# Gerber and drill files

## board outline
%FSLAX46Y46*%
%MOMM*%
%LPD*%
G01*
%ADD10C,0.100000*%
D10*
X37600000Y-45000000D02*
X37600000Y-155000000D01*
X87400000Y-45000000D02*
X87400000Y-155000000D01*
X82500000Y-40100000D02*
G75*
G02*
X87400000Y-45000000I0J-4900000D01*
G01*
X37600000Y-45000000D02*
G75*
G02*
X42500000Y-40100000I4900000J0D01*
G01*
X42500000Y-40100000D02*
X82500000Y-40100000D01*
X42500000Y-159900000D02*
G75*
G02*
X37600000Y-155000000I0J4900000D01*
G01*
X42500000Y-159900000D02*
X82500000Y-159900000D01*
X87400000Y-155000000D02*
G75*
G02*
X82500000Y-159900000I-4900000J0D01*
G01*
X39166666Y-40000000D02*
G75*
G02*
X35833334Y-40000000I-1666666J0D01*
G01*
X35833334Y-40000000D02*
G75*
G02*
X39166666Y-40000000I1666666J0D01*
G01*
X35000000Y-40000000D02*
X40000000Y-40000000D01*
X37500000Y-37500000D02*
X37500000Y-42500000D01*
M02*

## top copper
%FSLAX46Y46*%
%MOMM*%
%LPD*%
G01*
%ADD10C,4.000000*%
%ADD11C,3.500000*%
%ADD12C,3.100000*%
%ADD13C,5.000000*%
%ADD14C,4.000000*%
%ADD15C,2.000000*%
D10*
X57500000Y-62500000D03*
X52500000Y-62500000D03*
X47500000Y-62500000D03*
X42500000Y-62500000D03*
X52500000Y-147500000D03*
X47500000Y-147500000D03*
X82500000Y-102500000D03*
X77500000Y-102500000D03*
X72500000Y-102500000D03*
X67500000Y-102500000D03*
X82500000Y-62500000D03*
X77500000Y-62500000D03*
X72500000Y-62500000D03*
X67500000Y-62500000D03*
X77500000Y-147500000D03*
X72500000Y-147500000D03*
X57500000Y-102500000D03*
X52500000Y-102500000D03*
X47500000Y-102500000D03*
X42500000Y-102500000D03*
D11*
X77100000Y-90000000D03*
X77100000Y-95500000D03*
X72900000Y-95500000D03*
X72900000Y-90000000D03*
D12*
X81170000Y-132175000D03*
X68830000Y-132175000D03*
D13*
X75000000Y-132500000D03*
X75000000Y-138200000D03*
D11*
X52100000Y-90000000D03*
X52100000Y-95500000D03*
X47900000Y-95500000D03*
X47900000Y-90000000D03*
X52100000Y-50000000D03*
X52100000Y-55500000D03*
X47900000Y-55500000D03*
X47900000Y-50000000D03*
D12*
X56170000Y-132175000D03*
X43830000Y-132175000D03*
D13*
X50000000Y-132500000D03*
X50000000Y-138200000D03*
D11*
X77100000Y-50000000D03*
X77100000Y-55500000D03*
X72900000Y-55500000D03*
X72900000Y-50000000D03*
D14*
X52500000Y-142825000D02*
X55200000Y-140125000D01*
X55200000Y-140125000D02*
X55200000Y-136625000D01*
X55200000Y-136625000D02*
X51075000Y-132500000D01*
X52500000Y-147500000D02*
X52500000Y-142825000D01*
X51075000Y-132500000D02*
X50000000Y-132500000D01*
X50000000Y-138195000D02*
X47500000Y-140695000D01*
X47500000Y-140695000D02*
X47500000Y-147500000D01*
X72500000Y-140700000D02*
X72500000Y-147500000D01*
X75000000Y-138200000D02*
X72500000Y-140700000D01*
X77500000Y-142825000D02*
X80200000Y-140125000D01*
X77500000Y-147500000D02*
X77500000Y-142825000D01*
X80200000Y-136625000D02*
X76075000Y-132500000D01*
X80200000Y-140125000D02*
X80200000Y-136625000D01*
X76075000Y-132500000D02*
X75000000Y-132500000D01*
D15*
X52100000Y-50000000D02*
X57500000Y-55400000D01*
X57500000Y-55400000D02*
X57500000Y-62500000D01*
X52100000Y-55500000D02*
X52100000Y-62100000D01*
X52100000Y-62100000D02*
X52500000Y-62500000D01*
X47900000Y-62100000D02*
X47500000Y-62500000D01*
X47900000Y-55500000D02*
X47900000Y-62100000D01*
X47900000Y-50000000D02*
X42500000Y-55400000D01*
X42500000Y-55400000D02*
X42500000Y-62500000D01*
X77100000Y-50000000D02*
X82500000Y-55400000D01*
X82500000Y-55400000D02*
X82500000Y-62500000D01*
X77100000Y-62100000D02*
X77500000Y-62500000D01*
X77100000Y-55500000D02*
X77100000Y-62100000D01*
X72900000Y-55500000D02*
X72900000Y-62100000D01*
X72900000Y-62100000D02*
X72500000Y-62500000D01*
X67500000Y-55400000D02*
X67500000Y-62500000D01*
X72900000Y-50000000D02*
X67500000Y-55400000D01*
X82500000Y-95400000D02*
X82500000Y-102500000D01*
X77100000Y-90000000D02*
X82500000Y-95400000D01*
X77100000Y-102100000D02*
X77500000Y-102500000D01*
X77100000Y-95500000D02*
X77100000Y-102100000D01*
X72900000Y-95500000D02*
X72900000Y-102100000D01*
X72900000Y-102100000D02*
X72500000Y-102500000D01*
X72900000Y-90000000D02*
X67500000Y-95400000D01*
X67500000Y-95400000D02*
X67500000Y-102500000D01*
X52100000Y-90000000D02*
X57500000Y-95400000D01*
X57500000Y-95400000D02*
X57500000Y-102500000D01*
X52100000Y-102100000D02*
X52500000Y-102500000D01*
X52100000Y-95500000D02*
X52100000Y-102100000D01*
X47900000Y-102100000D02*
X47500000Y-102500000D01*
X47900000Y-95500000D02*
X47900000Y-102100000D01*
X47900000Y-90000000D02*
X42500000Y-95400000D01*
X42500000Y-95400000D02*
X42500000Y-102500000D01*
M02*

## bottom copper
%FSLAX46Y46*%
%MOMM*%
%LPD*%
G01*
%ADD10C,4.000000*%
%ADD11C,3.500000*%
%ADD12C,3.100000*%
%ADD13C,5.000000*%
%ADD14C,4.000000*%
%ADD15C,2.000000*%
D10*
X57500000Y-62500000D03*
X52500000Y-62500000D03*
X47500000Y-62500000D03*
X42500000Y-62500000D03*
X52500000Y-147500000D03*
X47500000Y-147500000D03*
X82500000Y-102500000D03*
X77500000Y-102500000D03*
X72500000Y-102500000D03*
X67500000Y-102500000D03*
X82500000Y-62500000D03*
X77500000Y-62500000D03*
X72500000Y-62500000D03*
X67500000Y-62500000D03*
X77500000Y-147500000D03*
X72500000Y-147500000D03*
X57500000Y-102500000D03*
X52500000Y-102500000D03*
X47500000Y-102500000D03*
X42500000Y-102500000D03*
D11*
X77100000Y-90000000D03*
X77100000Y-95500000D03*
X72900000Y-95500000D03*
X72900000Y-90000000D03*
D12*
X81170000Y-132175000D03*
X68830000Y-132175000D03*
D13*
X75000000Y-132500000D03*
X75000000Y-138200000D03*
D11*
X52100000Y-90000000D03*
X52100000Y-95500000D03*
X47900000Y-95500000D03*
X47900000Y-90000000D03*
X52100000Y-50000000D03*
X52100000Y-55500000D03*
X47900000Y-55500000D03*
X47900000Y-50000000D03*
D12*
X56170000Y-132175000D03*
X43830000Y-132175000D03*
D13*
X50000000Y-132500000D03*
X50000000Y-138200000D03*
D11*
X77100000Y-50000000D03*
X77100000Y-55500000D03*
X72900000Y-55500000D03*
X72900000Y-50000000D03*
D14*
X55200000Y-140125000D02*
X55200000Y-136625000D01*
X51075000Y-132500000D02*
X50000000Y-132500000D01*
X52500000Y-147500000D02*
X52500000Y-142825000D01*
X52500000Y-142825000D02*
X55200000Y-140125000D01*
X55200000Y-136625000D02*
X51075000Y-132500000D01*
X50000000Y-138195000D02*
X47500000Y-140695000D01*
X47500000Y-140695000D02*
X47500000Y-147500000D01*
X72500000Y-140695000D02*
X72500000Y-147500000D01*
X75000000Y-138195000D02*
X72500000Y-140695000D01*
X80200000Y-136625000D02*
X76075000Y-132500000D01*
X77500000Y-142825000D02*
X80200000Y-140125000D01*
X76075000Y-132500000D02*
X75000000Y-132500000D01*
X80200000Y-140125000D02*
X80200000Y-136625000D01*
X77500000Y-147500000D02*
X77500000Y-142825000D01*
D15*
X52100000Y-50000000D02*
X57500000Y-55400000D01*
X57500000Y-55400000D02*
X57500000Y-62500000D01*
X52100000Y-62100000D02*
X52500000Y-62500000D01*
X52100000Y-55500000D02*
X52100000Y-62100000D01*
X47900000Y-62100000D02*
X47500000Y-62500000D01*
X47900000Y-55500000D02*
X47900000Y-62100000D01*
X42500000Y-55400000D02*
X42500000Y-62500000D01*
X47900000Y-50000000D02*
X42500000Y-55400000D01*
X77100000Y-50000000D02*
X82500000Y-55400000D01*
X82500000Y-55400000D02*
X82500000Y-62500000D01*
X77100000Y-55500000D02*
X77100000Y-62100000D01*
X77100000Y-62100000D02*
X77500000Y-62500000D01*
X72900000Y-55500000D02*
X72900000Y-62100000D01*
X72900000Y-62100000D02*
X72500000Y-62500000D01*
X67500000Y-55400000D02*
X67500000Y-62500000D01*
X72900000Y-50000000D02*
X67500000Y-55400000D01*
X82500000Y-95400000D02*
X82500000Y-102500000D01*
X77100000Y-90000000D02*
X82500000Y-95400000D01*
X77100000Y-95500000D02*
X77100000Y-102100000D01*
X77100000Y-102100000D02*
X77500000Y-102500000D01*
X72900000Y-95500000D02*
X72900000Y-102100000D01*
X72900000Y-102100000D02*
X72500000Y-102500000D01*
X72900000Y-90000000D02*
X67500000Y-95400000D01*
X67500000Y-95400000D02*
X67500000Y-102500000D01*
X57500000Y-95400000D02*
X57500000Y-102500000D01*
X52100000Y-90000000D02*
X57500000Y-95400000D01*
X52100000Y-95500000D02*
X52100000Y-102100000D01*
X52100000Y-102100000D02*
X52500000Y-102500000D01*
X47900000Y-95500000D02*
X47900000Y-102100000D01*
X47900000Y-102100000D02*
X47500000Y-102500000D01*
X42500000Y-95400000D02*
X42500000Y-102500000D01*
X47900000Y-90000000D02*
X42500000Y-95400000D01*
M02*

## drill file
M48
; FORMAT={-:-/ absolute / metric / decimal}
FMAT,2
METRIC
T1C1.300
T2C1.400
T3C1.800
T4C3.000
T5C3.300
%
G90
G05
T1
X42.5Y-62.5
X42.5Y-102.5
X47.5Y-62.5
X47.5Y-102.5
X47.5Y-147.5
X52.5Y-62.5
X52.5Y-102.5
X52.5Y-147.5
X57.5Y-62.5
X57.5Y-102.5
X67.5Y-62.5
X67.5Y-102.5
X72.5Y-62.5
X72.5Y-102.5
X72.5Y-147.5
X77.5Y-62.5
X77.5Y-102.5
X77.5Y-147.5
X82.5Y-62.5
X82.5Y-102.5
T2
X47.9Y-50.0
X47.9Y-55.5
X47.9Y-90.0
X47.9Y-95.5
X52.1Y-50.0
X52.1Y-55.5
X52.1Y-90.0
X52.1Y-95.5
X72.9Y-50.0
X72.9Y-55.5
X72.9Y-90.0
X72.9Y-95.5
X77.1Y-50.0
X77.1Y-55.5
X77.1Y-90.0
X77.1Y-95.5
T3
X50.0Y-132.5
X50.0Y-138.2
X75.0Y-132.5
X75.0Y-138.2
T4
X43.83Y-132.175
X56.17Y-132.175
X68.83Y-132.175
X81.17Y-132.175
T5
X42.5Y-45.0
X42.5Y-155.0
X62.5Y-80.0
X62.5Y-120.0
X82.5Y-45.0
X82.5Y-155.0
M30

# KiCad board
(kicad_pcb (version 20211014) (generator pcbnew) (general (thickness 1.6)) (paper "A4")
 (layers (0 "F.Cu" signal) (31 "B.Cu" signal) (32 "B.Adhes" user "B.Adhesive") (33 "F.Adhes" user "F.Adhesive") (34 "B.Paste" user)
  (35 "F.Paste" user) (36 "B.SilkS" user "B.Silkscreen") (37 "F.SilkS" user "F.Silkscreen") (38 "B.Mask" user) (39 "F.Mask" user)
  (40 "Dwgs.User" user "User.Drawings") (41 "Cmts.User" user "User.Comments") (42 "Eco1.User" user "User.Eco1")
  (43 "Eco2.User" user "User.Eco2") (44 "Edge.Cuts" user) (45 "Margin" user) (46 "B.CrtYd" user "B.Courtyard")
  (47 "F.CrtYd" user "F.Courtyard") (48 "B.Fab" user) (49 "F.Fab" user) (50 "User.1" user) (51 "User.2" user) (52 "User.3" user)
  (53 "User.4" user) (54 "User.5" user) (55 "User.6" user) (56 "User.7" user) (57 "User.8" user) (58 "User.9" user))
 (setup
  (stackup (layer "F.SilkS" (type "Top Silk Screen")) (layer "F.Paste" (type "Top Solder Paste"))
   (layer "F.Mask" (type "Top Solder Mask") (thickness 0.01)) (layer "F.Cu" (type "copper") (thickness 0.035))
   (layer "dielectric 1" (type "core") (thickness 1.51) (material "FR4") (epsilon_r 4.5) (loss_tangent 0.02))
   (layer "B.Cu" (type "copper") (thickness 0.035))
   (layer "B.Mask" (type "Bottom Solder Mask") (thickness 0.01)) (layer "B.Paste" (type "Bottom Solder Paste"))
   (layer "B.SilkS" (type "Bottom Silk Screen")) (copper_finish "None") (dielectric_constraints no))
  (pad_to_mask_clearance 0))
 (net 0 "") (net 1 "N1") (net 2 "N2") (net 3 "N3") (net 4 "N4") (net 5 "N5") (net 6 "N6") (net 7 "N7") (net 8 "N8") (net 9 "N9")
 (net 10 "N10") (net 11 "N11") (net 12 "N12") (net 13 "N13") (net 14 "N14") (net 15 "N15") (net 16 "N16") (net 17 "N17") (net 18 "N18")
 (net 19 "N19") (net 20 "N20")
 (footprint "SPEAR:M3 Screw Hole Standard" (layer "F.Cu") (at 62.5 120)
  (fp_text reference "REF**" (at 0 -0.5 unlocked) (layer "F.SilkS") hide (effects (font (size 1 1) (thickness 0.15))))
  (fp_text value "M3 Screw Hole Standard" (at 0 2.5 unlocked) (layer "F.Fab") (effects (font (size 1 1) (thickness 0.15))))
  (pad "" np_thru_hole circle (at 0 0) (size 3.3 3.3) (drill 3.3) (layers F&B.Cu *.Mask)))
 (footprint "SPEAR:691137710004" (layer "F.Cu") (at 50 62.5)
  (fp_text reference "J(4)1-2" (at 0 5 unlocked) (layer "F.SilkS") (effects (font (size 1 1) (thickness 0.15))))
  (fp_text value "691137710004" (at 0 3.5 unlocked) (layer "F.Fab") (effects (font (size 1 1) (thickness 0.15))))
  (pad "1" thru_hole circle (at 7.5 0) (size 4 4) (drill 1.3) (layers *.Cu *.Mask) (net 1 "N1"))
  (pad "2" thru_hole circle (at 2.5 0) (size 4 4) (drill 1.3) (layers *.Cu *.Mask) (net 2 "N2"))
  (pad "3" thru_hole circle (at -2.5 0) (size 4 4) (drill 1.3) (layers *.Cu *.Mask) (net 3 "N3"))
  (pad "4" thru_hole circle (at -7.5 0) (size 4 4) (drill 1.3) (layers *.Cu *.Mask) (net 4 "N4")))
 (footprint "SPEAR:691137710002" (layer "F.Cu") (at 50 147.5)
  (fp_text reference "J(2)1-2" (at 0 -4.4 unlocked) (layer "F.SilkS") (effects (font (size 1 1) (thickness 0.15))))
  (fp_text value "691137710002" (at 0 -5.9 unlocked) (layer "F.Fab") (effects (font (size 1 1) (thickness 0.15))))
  (pad "1" thru_hole circle (at 2.5 0) (size 4 4) (drill 1.3) (layers *.Cu *.Mask) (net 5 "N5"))
  (pad "2" thru_hole circle (at -2.5 0) (size 4 4) (drill 1.3) (layers *.Cu *.Mask) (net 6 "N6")))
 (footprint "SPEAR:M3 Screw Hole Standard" (layer "F.Cu") (at 42.5 155)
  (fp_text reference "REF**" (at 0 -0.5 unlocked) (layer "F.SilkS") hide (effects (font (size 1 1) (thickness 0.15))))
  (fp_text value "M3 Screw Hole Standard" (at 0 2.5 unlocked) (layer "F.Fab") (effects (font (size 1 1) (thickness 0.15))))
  (pad "" np_thru_hole circle (at 0 0) (size 3.3 3.3) (drill 3.3) (layers F&B.Cu *.Mask)))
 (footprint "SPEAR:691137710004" (layer "F.Cu") (at 75 102.5)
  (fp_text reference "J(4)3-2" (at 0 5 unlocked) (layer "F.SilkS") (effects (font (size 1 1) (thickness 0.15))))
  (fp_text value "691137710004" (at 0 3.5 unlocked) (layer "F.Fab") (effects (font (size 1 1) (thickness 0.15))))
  (pad "1" thru_hole circle (at 7.5 0) (size 4 4) (drill 1.3) (layers *.Cu *.Mask) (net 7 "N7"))
  (pad "2" thru_hole circle (at 2.5 0) (size 4 4) (drill 1.3) (layers *.Cu *.Mask) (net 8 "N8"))
  (pad "3" thru_hole circle (at -2.5 0) (size 4 4) (drill 1.3) (layers *.Cu *.Mask) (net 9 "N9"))
  (pad "4" thru_hole circle (at -7.5 0) (size 4 4) (drill 1.3) (layers *.Cu *.Mask) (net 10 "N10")))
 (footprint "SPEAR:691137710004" (layer "F.Cu") (at 75 62.5)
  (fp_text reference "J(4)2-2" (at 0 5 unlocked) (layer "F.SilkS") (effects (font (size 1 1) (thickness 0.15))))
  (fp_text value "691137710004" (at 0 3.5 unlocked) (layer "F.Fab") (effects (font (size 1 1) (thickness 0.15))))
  (pad "1" thru_hole circle (at 7.5 0) (size 4 4) (drill 1.3) (layers *.Cu *.Mask) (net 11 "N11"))
  (pad "2" thru_hole circle (at 2.5 0) (size 4 4) (drill 1.3) (layers *.Cu *.Mask) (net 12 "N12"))
  (pad "3" thru_hole circle (at -2.5 0) (size 4 4) (drill 1.3) (layers *.Cu *.Mask) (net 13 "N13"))
  (pad "4" thru_hole circle (at -7.5 0) (size 4 4) (drill 1.3) (layers *.Cu *.Mask) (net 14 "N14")))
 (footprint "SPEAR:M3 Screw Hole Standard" (layer "F.Cu") (at 62.5 80)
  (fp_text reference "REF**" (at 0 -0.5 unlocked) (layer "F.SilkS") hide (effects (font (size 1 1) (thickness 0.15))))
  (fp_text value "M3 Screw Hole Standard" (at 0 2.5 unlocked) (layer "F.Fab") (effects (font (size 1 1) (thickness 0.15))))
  (pad "" np_thru_hole circle (at 0 0) (size 3.3 3.3) (drill 3.3) (layers F&B.Cu *.Mask)))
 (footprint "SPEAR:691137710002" (layer "F.Cu") (at 75 147.5)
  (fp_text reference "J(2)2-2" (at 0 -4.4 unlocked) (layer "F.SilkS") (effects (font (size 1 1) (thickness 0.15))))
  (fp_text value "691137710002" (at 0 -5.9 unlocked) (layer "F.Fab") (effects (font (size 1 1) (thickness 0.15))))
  (pad "1" thru_hole circle (at 2.5 0) (size 4 4) (drill 1.3) (layers *.Cu *.Mask) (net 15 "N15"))
  (pad "2" thru_hole circle (at -2.5 0) (size 4 4) (drill 1.3) (layers *.Cu *.Mask) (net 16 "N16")))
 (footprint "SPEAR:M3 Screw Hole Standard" (layer "F.Cu") (at 82.5 45)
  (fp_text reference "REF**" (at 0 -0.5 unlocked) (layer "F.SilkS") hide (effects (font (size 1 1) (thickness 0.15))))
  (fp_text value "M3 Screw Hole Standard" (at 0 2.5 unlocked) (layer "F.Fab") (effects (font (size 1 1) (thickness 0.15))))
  (pad "" np_thru_hole circle (at 0 0) (size 3.3 3.3) (drill 3.3) (layers F&B.Cu *.Mask)))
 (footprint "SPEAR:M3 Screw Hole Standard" (layer "F.Cu") (at 42.5 45)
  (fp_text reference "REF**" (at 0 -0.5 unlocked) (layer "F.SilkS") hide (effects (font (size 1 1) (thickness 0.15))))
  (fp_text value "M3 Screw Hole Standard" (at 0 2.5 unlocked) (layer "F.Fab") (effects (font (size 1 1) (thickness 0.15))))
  (pad "" np_thru_hole circle (at 0 0) (size 3.3 3.3) (drill 3.3) (layers F&B.Cu *.Mask)))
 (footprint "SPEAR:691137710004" (layer "F.Cu") (at 50 102.5)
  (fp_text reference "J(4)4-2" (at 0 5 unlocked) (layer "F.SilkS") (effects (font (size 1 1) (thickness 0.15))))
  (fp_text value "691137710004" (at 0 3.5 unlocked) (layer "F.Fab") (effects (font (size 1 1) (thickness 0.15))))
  (pad "1" thru_hole circle (at 7.5 0) (size 4 4) (drill 1.3) (layers *.Cu *.Mask) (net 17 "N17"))
  (pad "2" thru_hole circle (at 2.5 0) (size 4 4) (drill 1.3) (layers *.Cu *.Mask) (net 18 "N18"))
  (pad "3" thru_hole circle (at -2.5 0) (size 4 4) (drill 1.3) (layers *.Cu *.Mask) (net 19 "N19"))
  (pad "4" thru_hole circle (at -7.5 0) (size 4 4) (drill 1.3) (layers *.Cu *.Mask) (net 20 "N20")))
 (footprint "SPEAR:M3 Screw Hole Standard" (layer "F.Cu") (at 82.5 155)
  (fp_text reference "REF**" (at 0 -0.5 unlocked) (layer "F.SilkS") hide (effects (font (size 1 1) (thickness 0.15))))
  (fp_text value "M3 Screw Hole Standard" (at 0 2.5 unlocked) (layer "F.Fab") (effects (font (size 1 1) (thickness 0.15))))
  (pad "" np_thru_hole circle (at 0 0) (size 3.3 3.3) (drill 3.3) (layers F&B.Cu *.Mask)))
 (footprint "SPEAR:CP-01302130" (layer "B.Cu") (at 75 90 180)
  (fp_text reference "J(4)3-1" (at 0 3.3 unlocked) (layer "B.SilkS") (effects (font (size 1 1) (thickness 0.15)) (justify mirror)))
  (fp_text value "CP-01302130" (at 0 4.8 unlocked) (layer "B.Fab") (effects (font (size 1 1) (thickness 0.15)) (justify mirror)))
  (pad "1" thru_hole circle (at -2.1 0 180) (size 3.5 3.5) (drill 1.4) (layers *.Cu *.Mask) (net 7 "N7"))
  (pad "2" thru_hole circle (at -2.1 -5.5 180) (size 3.5 3.5) (drill 1.4) (layers *.Cu *.Mask) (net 8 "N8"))
  (pad "3" thru_hole circle (at 2.1 -5.5 180) (size 3.5 3.5) (drill 1.4) (layers *.Cu *.Mask) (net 9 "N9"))
  (pad "4" thru_hole circle (at 2.1 0 180) (size 3.5 3.5) (drill 1.4) (layers *.Cu *.Mask) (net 10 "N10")))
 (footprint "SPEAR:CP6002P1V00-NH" (layer "B.Cu") (at 75 132.5 180)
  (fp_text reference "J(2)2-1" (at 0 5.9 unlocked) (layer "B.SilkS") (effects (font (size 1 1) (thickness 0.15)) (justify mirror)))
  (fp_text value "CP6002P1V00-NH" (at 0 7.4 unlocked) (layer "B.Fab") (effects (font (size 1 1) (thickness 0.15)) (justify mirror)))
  (pad "" np_thru_hole circle (at -6.17 0.325 180) (size 3.1 3.1) (drill 3) (layers F&B.Cu *.Mask))
  (pad "" np_thru_hole circle (at 6.17 0.325 180) (size 3.1 3.1) (drill 3) (layers F&B.Cu *.Mask))
  (pad "1" thru_hole circle (at 0 0 180) (size 5 5) (drill 1.8) (layers *.Cu *.Mask) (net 15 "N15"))
  (pad "2" thru_hole circle (at 0 -5.7 180) (size 5 5) (drill 1.8) (layers *.Cu *.Mask) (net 16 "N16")))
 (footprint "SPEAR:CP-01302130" (layer "B.Cu") (at 50 90 180)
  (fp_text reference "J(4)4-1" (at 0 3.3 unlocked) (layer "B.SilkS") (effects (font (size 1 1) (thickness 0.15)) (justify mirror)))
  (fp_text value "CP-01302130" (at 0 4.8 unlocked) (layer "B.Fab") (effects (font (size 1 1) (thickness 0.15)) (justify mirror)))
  (pad "1" thru_hole circle (at -2.1 0 180) (size 3.5 3.5) (drill 1.4) (layers *.Cu *.Mask) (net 17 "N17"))
  (pad "2" thru_hole circle (at -2.1 -5.5 180) (size 3.5 3.5) (drill 1.4) (layers *.Cu *.Mask) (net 18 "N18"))
  (pad "3" thru_hole circle (at 2.1 -5.5 180) (size 3.5 3.5) (drill 1.4) (layers *.Cu *.Mask) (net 19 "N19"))
  (pad "4" thru_hole circle (at 2.1 0 180) (size 3.5 3.5) (drill 1.4) (layers *.Cu *.Mask) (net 20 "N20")))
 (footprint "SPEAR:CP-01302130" (layer "B.Cu") (at 50 50 180)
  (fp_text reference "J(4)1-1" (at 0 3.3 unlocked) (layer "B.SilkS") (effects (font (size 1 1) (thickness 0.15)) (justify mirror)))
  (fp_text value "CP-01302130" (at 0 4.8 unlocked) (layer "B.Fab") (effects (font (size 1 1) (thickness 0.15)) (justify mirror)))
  (pad "1" thru_hole circle (at -2.1 0 180) (size 3.5 3.5) (drill 1.4) (layers *.Cu *.Mask) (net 1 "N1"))
  (pad "2" thru_hole circle (at -2.1 -5.5 180) (size 3.5 3.5) (drill 1.4) (layers *.Cu *.Mask) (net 2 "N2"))
  (pad "3" thru_hole circle (at 2.1 -5.5 180) (size 3.5 3.5) (drill 1.4) (layers *.Cu *.Mask) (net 3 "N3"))
  (pad "4" thru_hole circle (at 2.1 0 180) (size 3.5 3.5) (drill 1.4) (layers *.Cu *.Mask) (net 4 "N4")))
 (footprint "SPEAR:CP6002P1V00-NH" (layer "B.Cu") (at 50 132.5 180)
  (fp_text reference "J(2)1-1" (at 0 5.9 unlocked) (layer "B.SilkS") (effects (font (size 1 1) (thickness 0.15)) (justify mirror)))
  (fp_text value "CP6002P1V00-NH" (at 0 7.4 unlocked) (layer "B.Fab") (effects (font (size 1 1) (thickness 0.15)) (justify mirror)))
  (pad "" np_thru_hole circle (at -6.17 0.325 180) (size 3.1 3.1) (drill 3) (layers F&B.Cu *.Mask))
  (pad "" np_thru_hole circle (at 6.17 0.325 180) (size 3.1 3.1) (drill 3) (layers F&B.Cu *.Mask))
  (pad "1" thru_hole circle (at 0 0 180) (size 5 5) (drill 1.8) (layers *.Cu *.Mask) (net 5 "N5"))
  (pad "2" thru_hole circle (at 0 -5.7 180) (size 5 5) (drill 1.8) (layers *.Cu *.Mask) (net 6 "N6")))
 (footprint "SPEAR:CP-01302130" (layer "B.Cu") (at 75 50 180)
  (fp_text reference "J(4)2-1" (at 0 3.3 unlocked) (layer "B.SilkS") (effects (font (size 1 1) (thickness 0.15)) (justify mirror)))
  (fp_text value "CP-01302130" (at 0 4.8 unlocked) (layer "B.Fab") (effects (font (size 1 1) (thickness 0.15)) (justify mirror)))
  (pad "1" thru_hole circle (at -2.1 0 180) (size 3.5 3.5) (drill 1.4) (layers *.Cu *.Mask) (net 11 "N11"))
  (pad "2" thru_hole circle (at -2.1 -5.5 180) (size 3.5 3.5) (drill 1.4) (layers *.Cu *.Mask) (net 12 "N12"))
  (pad "3" thru_hole circle (at 2.1 -5.5 180) (size 3.5 3.5) (drill 1.4) (layers *.Cu *.Mask) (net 13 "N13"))
  (pad "4" thru_hole circle (at 2.1 0 180) (size 3.5 3.5) (drill 1.4) (layers *.Cu *.Mask) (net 14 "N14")))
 (gr_line (start 37.6 45) (end 37.6 155) (layer "Edge.Cuts") (width 0.1))
 (gr_line (start 87.4 45) (end 87.4 155) (layer "Edge.Cuts") (width 0.1))
 (gr_arc (start 82.5 40.1) (mid 85.964823 41.535177) (end 87.4 45) (layer "Edge.Cuts") (width 0.1))
 (gr_arc (start 37.6 45) (mid 39.035177 41.535177) (end 42.5 40.1) (layer "Edge.Cuts") (width 0.1))
 (gr_line (start 42.5 40.1) (end 82.5 40.1) (layer "Edge.Cuts") (width 0.1))
 (gr_arc (start 42.5 159.9) (mid 39.035177 158.464823) (end 37.6 155) (layer "Edge.Cuts") (width 0.1))
 (gr_line (start 42.5 159.9) (end 82.5 159.9) (layer "Edge.Cuts") (width 0.1))
 (gr_arc (start 87.4 155) (mid 85.964823 158.464823) (end 82.5 159.9) (layer "Edge.Cuts") (width 0.1))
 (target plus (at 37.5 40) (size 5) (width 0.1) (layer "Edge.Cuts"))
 (segment (start 52.5 142.825) (end 55.2 140.125) (width 4) (layer "F.Cu") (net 5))
 (segment (start 55.2 140.125) (end 55.2 136.625) (width 4) (layer "F.Cu") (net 5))
 (segment (start 55.2 136.625) (end 51.075 132.5) (width 4) (layer "F.Cu") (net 5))
 (segment (start 52.5 147.5) (end 52.5 142.825) (width 4) (layer "F.Cu") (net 5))
 (segment (start 51.075 132.5) (end 50 132.5) (width 4) (layer "F.Cu") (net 5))
 (segment (start 55.2 140.125) (end 55.2 136.625) (width 4) (layer "B.Cu") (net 5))
 (segment (start 51.075 132.5) (end 50 132.5) (width 4) (layer "B.Cu") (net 5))
 (segment (start 52.5 147.5) (end 52.5 142.825) (width 4) (layer "B.Cu") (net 5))
 (segment (start 52.5 142.825) (end 55.2 140.125) (width 4) (layer "B.Cu") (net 5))
 (segment (start 55.2 136.625) (end 51.075 132.5) (width 4) (layer "B.Cu") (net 5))
 (segment (start 50 138.195) (end 47.5 140.695) (width 4) (layer "F.Cu") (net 6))
 (segment (start 47.5 140.695) (end 47.5 147.5) (width 4) (layer "F.Cu") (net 6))
 (segment (start 50 138.195) (end 47.5 140.695) (width 4) (layer "B.Cu") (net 6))
 (segment (start 47.5 140.695) (end 47.5 147.5) (width 4) (layer "B.Cu") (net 6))
 (segment (start 72.5 140.7) (end 72.5 147.5) (width 4) (layer "F.Cu") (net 16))
 (segment (start 75 138.2) (end 72.5 140.7) (width 4) (layer "F.Cu") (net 16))
 (segment (start 72.5 140.695) (end 72.5 147.5) (width 4) (layer "B.Cu") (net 16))
 (segment (start 75 138.195) (end 72.5 140.695) (width 4) (layer "B.Cu") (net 16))
 (segment (start 77.5 142.825) (end 80.2 140.125) (width 4) (layer "F.Cu") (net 15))
 (segment (start 77.5 147.5) (end 77.5 142.825) (width 4) (layer "F.Cu") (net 15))
 (segment (start 80.2 136.625) (end 76.075 132.5) (width 4) (layer "F.Cu") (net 15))
 (segment (start 80.2 140.125) (end 80.2 136.625) (width 4) (layer "F.Cu") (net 15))
 (segment (start 76.075 132.5) (end 75 132.5) (width 4) (layer "F.Cu") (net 15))
 (segment (start 80.2 136.625) (end 76.075 132.5) (width 4) (layer "B.Cu") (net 15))
 (segment (start 77.5 142.825) (end 80.2 140.125) (width 4) (layer "B.Cu") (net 15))
 (segment (start 76.075 132.5) (end 75 132.5) (width 4) (layer "B.Cu") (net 15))
 (segment (start 80.2 140.125) (end 80.2 136.625) (width 4) (layer "B.Cu") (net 15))
 (segment (start 77.5 147.5) (end 77.5 142.825) (width 4) (layer "B.Cu") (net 15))
 (segment (start 52.1 50) (end 57.5 55.4) (width 2) (layer "F.Cu") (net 1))
 (segment (start 57.5 55.4) (end 57.5 62.5) (width 2) (layer "F.Cu") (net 1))
 (segment (start 52.1 50) (end 57.5 55.4) (width 2) (layer "B.Cu") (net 1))
 (segment (start 57.5 55.4) (end 57.5 62.5) (width 2) (layer "B.Cu") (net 1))
 (segment (start 52.1 55.5) (end 52.1 62.1) (width 2) (layer "F.Cu") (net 2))
 (segment (start 52.1 62.1) (end 52.5 62.5) (width 2) (layer "F.Cu") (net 2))
 (segment (start 52.1 62.1) (end 52.5 62.5) (width 2) (layer "B.Cu") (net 2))
 (segment (start 52.1 55.5) (end 52.1 62.1) (width 2) (layer "B.Cu") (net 2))
 (segment (start 47.9 62.1) (end 47.5 62.5) (width 2) (layer "F.Cu") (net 3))
 (segment (start 47.9 55.5) (end 47.9 62.1) (width 2) (layer "F.Cu") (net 3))
 (segment (start 47.9 62.1) (end 47.5 62.5) (width 2) (layer "B.Cu") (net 3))
 (segment (start 47.9 55.5) (end 47.9 62.1) (width 2) (layer "B.Cu") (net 3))
 (segment (start 47.9 50) (end 42.5 55.4) (width 2) (layer "F.Cu") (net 4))
 (segment (start 42.5 55.4) (end 42.5 62.5) (width 2) (layer "F.Cu") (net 4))
 (segment (start 42.5 55.4) (end 42.5 62.5) (width 2) (layer "B.Cu") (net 4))
 (segment (start 47.9 50) (end 42.5 55.4) (width 2) (layer "B.Cu") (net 4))
 (segment (start 77.1 50) (end 82.5 55.4) (width 2) (layer "F.Cu") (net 11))
 (segment (start 82.5 55.4) (end 82.5 62.5) (width 2) (layer "F.Cu") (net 11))
 (segment (start 77.1 50) (end 82.5 55.4) (width 2) (layer "B.Cu") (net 11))
 (segment (start 82.5 55.4) (end 82.5 62.5) (width 2) (layer "B.Cu") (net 11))
 (segment (start 77.1 62.1) (end 77.5 62.5) (width 2) (layer "F.Cu") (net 12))
 (segment (start 77.1 55.5) (end 77.1 62.1) (width 2) (layer "F.Cu") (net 12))
 (segment (start 77.1 55.5) (end 77.1 62.1) (width 2) (layer "B.Cu") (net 12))
 (segment (start 77.1 62.1) (end 77.5 62.5) (width 2) (layer "B.Cu") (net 12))
 (segment (start 72.9 55.5) (end 72.9 62.1) (width 2) (layer "F.Cu") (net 13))
 (segment (start 72.9 62.1) (end 72.5 62.5) (width 2) (layer "F.Cu") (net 13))
 (segment (start 72.9 55.5) (end 72.9 62.1) (width 2) (layer "B.Cu") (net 13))
 (segment (start 72.9 62.1) (end 72.5 62.5) (width 2) (layer "B.Cu") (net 13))
 (segment (start 67.5 55.4) (end 67.5 62.5) (width 2) (layer "F.Cu") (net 14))
 (segment (start 72.9 50) (end 67.5 55.4) (width 2) (layer "F.Cu") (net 14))
 (segment (start 67.5 55.4) (end 67.5 62.5) (width 2) (layer "B.Cu") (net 14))
 (segment (start 72.9 50) (end 67.5 55.4) (width 2) (layer "B.Cu") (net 14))
 (segment (start 82.5 95.4) (end 82.5 102.5) (width 2) (layer "F.Cu") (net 7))
 (segment (start 77.1 90) (end 82.5 95.4) (width 2) (layer "F.Cu") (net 7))
 (segment (start 82.5 95.4) (end 82.5 102.5) (width 2) (layer "B.Cu") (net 7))
 (segment (start 77.1 90) (end 82.5 95.4) (width 2) (layer "B.Cu") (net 7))
 (segment (start 77.1 102.1) (end 77.5 102.5) (width 2) (layer "F.Cu") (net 8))
 (segment (start 77.1 95.5) (end 77.1 102.1) (width 2) (layer "F.Cu") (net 8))
 (segment (start 77.1 95.5) (end 77.1 102.1) (width 2) (layer "B.Cu") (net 8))
 (segment (start 77.1 102.1) (end 77.5 102.5) (width 2) (layer "B.Cu") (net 8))
 (segment (start 72.9 95.5) (end 72.9 102.1) (width 2) (layer "F.Cu") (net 9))
 (segment (start 72.9 102.1) (end 72.5 102.5) (width 2) (layer "F.Cu") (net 9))
 (segment (start 72.9 95.5) (end 72.9 102.1) (width 2) (layer "B.Cu") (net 9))
 (segment (start 72.9 102.1) (end 72.5 102.5) (width 2) (layer "B.Cu") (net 9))
 (segment (start 72.9 90) (end 67.5 95.4) (width 2) (layer "F.Cu") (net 10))
 (segment (start 67.5 95.4) (end 67.5 102.5) (width 2) (layer "F.Cu") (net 10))
 (segment (start 72.9 90) (end 67.5 95.4) (width 2) (layer "B.Cu") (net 10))
 (segment (start 67.5 95.4) (end 67.5 102.5) (width 2) (layer "B.Cu") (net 10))
 (segment (start 52.1 90) (end 57.5 95.4) (width 2) (layer "F.Cu") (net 17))
 (segment (start 57.5 95.4) (end 57.5 102.5) (width 2) (layer "F.Cu") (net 17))
 (segment (start 57.5 95.4) (end 57.5 102.5) (width 2) (layer "B.Cu") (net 17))
 (segment (start 52.1 90) (end 57.5 95.4) (width 2) (layer "B.Cu") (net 17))
 (segment (start 52.1 102.1) (end 52.5 102.5) (width 2) (layer "F.Cu") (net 18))
 (segment (start 52.1 95.5) (end 52.1 102.1) (width 2) (layer "F.Cu") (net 18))
 (segment (start 52.1 95.5) (end 52.1 102.1) (width 2) (layer "B.Cu") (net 18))
 (segment (start 52.1 102.1) (end 52.5 102.5) (width 2) (layer "B.Cu") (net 18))
 (segment (start 47.9 102.1) (end 47.5 102.5) (width 2) (layer "F.Cu") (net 19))
 (segment (start 47.9 95.5) (end 47.9 102.1) (width 2) (layer "F.Cu") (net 19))
 (segment (start 47.9 95.5) (end 47.9 102.1) (width 2) (layer "B.Cu") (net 19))
 (segment (start 47.9 102.1) (end 47.5 102.5) (width 2) (layer "B.Cu") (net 19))
 (segment (start 47.9 90) (end 42.5 95.4) (width 2) (layer "F.Cu") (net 20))
 (segment (start 42.5 95.4) (end 42.5 102.5) (width 2) (layer "F.Cu") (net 20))
 (segment (start 42.5 95.4) (end 42.5 102.5) (width 2) (layer "B.Cu") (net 20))
 (segment (start 47.9 90) (end 42.5 95.4) (width 2) (layer "B.Cu") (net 20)))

